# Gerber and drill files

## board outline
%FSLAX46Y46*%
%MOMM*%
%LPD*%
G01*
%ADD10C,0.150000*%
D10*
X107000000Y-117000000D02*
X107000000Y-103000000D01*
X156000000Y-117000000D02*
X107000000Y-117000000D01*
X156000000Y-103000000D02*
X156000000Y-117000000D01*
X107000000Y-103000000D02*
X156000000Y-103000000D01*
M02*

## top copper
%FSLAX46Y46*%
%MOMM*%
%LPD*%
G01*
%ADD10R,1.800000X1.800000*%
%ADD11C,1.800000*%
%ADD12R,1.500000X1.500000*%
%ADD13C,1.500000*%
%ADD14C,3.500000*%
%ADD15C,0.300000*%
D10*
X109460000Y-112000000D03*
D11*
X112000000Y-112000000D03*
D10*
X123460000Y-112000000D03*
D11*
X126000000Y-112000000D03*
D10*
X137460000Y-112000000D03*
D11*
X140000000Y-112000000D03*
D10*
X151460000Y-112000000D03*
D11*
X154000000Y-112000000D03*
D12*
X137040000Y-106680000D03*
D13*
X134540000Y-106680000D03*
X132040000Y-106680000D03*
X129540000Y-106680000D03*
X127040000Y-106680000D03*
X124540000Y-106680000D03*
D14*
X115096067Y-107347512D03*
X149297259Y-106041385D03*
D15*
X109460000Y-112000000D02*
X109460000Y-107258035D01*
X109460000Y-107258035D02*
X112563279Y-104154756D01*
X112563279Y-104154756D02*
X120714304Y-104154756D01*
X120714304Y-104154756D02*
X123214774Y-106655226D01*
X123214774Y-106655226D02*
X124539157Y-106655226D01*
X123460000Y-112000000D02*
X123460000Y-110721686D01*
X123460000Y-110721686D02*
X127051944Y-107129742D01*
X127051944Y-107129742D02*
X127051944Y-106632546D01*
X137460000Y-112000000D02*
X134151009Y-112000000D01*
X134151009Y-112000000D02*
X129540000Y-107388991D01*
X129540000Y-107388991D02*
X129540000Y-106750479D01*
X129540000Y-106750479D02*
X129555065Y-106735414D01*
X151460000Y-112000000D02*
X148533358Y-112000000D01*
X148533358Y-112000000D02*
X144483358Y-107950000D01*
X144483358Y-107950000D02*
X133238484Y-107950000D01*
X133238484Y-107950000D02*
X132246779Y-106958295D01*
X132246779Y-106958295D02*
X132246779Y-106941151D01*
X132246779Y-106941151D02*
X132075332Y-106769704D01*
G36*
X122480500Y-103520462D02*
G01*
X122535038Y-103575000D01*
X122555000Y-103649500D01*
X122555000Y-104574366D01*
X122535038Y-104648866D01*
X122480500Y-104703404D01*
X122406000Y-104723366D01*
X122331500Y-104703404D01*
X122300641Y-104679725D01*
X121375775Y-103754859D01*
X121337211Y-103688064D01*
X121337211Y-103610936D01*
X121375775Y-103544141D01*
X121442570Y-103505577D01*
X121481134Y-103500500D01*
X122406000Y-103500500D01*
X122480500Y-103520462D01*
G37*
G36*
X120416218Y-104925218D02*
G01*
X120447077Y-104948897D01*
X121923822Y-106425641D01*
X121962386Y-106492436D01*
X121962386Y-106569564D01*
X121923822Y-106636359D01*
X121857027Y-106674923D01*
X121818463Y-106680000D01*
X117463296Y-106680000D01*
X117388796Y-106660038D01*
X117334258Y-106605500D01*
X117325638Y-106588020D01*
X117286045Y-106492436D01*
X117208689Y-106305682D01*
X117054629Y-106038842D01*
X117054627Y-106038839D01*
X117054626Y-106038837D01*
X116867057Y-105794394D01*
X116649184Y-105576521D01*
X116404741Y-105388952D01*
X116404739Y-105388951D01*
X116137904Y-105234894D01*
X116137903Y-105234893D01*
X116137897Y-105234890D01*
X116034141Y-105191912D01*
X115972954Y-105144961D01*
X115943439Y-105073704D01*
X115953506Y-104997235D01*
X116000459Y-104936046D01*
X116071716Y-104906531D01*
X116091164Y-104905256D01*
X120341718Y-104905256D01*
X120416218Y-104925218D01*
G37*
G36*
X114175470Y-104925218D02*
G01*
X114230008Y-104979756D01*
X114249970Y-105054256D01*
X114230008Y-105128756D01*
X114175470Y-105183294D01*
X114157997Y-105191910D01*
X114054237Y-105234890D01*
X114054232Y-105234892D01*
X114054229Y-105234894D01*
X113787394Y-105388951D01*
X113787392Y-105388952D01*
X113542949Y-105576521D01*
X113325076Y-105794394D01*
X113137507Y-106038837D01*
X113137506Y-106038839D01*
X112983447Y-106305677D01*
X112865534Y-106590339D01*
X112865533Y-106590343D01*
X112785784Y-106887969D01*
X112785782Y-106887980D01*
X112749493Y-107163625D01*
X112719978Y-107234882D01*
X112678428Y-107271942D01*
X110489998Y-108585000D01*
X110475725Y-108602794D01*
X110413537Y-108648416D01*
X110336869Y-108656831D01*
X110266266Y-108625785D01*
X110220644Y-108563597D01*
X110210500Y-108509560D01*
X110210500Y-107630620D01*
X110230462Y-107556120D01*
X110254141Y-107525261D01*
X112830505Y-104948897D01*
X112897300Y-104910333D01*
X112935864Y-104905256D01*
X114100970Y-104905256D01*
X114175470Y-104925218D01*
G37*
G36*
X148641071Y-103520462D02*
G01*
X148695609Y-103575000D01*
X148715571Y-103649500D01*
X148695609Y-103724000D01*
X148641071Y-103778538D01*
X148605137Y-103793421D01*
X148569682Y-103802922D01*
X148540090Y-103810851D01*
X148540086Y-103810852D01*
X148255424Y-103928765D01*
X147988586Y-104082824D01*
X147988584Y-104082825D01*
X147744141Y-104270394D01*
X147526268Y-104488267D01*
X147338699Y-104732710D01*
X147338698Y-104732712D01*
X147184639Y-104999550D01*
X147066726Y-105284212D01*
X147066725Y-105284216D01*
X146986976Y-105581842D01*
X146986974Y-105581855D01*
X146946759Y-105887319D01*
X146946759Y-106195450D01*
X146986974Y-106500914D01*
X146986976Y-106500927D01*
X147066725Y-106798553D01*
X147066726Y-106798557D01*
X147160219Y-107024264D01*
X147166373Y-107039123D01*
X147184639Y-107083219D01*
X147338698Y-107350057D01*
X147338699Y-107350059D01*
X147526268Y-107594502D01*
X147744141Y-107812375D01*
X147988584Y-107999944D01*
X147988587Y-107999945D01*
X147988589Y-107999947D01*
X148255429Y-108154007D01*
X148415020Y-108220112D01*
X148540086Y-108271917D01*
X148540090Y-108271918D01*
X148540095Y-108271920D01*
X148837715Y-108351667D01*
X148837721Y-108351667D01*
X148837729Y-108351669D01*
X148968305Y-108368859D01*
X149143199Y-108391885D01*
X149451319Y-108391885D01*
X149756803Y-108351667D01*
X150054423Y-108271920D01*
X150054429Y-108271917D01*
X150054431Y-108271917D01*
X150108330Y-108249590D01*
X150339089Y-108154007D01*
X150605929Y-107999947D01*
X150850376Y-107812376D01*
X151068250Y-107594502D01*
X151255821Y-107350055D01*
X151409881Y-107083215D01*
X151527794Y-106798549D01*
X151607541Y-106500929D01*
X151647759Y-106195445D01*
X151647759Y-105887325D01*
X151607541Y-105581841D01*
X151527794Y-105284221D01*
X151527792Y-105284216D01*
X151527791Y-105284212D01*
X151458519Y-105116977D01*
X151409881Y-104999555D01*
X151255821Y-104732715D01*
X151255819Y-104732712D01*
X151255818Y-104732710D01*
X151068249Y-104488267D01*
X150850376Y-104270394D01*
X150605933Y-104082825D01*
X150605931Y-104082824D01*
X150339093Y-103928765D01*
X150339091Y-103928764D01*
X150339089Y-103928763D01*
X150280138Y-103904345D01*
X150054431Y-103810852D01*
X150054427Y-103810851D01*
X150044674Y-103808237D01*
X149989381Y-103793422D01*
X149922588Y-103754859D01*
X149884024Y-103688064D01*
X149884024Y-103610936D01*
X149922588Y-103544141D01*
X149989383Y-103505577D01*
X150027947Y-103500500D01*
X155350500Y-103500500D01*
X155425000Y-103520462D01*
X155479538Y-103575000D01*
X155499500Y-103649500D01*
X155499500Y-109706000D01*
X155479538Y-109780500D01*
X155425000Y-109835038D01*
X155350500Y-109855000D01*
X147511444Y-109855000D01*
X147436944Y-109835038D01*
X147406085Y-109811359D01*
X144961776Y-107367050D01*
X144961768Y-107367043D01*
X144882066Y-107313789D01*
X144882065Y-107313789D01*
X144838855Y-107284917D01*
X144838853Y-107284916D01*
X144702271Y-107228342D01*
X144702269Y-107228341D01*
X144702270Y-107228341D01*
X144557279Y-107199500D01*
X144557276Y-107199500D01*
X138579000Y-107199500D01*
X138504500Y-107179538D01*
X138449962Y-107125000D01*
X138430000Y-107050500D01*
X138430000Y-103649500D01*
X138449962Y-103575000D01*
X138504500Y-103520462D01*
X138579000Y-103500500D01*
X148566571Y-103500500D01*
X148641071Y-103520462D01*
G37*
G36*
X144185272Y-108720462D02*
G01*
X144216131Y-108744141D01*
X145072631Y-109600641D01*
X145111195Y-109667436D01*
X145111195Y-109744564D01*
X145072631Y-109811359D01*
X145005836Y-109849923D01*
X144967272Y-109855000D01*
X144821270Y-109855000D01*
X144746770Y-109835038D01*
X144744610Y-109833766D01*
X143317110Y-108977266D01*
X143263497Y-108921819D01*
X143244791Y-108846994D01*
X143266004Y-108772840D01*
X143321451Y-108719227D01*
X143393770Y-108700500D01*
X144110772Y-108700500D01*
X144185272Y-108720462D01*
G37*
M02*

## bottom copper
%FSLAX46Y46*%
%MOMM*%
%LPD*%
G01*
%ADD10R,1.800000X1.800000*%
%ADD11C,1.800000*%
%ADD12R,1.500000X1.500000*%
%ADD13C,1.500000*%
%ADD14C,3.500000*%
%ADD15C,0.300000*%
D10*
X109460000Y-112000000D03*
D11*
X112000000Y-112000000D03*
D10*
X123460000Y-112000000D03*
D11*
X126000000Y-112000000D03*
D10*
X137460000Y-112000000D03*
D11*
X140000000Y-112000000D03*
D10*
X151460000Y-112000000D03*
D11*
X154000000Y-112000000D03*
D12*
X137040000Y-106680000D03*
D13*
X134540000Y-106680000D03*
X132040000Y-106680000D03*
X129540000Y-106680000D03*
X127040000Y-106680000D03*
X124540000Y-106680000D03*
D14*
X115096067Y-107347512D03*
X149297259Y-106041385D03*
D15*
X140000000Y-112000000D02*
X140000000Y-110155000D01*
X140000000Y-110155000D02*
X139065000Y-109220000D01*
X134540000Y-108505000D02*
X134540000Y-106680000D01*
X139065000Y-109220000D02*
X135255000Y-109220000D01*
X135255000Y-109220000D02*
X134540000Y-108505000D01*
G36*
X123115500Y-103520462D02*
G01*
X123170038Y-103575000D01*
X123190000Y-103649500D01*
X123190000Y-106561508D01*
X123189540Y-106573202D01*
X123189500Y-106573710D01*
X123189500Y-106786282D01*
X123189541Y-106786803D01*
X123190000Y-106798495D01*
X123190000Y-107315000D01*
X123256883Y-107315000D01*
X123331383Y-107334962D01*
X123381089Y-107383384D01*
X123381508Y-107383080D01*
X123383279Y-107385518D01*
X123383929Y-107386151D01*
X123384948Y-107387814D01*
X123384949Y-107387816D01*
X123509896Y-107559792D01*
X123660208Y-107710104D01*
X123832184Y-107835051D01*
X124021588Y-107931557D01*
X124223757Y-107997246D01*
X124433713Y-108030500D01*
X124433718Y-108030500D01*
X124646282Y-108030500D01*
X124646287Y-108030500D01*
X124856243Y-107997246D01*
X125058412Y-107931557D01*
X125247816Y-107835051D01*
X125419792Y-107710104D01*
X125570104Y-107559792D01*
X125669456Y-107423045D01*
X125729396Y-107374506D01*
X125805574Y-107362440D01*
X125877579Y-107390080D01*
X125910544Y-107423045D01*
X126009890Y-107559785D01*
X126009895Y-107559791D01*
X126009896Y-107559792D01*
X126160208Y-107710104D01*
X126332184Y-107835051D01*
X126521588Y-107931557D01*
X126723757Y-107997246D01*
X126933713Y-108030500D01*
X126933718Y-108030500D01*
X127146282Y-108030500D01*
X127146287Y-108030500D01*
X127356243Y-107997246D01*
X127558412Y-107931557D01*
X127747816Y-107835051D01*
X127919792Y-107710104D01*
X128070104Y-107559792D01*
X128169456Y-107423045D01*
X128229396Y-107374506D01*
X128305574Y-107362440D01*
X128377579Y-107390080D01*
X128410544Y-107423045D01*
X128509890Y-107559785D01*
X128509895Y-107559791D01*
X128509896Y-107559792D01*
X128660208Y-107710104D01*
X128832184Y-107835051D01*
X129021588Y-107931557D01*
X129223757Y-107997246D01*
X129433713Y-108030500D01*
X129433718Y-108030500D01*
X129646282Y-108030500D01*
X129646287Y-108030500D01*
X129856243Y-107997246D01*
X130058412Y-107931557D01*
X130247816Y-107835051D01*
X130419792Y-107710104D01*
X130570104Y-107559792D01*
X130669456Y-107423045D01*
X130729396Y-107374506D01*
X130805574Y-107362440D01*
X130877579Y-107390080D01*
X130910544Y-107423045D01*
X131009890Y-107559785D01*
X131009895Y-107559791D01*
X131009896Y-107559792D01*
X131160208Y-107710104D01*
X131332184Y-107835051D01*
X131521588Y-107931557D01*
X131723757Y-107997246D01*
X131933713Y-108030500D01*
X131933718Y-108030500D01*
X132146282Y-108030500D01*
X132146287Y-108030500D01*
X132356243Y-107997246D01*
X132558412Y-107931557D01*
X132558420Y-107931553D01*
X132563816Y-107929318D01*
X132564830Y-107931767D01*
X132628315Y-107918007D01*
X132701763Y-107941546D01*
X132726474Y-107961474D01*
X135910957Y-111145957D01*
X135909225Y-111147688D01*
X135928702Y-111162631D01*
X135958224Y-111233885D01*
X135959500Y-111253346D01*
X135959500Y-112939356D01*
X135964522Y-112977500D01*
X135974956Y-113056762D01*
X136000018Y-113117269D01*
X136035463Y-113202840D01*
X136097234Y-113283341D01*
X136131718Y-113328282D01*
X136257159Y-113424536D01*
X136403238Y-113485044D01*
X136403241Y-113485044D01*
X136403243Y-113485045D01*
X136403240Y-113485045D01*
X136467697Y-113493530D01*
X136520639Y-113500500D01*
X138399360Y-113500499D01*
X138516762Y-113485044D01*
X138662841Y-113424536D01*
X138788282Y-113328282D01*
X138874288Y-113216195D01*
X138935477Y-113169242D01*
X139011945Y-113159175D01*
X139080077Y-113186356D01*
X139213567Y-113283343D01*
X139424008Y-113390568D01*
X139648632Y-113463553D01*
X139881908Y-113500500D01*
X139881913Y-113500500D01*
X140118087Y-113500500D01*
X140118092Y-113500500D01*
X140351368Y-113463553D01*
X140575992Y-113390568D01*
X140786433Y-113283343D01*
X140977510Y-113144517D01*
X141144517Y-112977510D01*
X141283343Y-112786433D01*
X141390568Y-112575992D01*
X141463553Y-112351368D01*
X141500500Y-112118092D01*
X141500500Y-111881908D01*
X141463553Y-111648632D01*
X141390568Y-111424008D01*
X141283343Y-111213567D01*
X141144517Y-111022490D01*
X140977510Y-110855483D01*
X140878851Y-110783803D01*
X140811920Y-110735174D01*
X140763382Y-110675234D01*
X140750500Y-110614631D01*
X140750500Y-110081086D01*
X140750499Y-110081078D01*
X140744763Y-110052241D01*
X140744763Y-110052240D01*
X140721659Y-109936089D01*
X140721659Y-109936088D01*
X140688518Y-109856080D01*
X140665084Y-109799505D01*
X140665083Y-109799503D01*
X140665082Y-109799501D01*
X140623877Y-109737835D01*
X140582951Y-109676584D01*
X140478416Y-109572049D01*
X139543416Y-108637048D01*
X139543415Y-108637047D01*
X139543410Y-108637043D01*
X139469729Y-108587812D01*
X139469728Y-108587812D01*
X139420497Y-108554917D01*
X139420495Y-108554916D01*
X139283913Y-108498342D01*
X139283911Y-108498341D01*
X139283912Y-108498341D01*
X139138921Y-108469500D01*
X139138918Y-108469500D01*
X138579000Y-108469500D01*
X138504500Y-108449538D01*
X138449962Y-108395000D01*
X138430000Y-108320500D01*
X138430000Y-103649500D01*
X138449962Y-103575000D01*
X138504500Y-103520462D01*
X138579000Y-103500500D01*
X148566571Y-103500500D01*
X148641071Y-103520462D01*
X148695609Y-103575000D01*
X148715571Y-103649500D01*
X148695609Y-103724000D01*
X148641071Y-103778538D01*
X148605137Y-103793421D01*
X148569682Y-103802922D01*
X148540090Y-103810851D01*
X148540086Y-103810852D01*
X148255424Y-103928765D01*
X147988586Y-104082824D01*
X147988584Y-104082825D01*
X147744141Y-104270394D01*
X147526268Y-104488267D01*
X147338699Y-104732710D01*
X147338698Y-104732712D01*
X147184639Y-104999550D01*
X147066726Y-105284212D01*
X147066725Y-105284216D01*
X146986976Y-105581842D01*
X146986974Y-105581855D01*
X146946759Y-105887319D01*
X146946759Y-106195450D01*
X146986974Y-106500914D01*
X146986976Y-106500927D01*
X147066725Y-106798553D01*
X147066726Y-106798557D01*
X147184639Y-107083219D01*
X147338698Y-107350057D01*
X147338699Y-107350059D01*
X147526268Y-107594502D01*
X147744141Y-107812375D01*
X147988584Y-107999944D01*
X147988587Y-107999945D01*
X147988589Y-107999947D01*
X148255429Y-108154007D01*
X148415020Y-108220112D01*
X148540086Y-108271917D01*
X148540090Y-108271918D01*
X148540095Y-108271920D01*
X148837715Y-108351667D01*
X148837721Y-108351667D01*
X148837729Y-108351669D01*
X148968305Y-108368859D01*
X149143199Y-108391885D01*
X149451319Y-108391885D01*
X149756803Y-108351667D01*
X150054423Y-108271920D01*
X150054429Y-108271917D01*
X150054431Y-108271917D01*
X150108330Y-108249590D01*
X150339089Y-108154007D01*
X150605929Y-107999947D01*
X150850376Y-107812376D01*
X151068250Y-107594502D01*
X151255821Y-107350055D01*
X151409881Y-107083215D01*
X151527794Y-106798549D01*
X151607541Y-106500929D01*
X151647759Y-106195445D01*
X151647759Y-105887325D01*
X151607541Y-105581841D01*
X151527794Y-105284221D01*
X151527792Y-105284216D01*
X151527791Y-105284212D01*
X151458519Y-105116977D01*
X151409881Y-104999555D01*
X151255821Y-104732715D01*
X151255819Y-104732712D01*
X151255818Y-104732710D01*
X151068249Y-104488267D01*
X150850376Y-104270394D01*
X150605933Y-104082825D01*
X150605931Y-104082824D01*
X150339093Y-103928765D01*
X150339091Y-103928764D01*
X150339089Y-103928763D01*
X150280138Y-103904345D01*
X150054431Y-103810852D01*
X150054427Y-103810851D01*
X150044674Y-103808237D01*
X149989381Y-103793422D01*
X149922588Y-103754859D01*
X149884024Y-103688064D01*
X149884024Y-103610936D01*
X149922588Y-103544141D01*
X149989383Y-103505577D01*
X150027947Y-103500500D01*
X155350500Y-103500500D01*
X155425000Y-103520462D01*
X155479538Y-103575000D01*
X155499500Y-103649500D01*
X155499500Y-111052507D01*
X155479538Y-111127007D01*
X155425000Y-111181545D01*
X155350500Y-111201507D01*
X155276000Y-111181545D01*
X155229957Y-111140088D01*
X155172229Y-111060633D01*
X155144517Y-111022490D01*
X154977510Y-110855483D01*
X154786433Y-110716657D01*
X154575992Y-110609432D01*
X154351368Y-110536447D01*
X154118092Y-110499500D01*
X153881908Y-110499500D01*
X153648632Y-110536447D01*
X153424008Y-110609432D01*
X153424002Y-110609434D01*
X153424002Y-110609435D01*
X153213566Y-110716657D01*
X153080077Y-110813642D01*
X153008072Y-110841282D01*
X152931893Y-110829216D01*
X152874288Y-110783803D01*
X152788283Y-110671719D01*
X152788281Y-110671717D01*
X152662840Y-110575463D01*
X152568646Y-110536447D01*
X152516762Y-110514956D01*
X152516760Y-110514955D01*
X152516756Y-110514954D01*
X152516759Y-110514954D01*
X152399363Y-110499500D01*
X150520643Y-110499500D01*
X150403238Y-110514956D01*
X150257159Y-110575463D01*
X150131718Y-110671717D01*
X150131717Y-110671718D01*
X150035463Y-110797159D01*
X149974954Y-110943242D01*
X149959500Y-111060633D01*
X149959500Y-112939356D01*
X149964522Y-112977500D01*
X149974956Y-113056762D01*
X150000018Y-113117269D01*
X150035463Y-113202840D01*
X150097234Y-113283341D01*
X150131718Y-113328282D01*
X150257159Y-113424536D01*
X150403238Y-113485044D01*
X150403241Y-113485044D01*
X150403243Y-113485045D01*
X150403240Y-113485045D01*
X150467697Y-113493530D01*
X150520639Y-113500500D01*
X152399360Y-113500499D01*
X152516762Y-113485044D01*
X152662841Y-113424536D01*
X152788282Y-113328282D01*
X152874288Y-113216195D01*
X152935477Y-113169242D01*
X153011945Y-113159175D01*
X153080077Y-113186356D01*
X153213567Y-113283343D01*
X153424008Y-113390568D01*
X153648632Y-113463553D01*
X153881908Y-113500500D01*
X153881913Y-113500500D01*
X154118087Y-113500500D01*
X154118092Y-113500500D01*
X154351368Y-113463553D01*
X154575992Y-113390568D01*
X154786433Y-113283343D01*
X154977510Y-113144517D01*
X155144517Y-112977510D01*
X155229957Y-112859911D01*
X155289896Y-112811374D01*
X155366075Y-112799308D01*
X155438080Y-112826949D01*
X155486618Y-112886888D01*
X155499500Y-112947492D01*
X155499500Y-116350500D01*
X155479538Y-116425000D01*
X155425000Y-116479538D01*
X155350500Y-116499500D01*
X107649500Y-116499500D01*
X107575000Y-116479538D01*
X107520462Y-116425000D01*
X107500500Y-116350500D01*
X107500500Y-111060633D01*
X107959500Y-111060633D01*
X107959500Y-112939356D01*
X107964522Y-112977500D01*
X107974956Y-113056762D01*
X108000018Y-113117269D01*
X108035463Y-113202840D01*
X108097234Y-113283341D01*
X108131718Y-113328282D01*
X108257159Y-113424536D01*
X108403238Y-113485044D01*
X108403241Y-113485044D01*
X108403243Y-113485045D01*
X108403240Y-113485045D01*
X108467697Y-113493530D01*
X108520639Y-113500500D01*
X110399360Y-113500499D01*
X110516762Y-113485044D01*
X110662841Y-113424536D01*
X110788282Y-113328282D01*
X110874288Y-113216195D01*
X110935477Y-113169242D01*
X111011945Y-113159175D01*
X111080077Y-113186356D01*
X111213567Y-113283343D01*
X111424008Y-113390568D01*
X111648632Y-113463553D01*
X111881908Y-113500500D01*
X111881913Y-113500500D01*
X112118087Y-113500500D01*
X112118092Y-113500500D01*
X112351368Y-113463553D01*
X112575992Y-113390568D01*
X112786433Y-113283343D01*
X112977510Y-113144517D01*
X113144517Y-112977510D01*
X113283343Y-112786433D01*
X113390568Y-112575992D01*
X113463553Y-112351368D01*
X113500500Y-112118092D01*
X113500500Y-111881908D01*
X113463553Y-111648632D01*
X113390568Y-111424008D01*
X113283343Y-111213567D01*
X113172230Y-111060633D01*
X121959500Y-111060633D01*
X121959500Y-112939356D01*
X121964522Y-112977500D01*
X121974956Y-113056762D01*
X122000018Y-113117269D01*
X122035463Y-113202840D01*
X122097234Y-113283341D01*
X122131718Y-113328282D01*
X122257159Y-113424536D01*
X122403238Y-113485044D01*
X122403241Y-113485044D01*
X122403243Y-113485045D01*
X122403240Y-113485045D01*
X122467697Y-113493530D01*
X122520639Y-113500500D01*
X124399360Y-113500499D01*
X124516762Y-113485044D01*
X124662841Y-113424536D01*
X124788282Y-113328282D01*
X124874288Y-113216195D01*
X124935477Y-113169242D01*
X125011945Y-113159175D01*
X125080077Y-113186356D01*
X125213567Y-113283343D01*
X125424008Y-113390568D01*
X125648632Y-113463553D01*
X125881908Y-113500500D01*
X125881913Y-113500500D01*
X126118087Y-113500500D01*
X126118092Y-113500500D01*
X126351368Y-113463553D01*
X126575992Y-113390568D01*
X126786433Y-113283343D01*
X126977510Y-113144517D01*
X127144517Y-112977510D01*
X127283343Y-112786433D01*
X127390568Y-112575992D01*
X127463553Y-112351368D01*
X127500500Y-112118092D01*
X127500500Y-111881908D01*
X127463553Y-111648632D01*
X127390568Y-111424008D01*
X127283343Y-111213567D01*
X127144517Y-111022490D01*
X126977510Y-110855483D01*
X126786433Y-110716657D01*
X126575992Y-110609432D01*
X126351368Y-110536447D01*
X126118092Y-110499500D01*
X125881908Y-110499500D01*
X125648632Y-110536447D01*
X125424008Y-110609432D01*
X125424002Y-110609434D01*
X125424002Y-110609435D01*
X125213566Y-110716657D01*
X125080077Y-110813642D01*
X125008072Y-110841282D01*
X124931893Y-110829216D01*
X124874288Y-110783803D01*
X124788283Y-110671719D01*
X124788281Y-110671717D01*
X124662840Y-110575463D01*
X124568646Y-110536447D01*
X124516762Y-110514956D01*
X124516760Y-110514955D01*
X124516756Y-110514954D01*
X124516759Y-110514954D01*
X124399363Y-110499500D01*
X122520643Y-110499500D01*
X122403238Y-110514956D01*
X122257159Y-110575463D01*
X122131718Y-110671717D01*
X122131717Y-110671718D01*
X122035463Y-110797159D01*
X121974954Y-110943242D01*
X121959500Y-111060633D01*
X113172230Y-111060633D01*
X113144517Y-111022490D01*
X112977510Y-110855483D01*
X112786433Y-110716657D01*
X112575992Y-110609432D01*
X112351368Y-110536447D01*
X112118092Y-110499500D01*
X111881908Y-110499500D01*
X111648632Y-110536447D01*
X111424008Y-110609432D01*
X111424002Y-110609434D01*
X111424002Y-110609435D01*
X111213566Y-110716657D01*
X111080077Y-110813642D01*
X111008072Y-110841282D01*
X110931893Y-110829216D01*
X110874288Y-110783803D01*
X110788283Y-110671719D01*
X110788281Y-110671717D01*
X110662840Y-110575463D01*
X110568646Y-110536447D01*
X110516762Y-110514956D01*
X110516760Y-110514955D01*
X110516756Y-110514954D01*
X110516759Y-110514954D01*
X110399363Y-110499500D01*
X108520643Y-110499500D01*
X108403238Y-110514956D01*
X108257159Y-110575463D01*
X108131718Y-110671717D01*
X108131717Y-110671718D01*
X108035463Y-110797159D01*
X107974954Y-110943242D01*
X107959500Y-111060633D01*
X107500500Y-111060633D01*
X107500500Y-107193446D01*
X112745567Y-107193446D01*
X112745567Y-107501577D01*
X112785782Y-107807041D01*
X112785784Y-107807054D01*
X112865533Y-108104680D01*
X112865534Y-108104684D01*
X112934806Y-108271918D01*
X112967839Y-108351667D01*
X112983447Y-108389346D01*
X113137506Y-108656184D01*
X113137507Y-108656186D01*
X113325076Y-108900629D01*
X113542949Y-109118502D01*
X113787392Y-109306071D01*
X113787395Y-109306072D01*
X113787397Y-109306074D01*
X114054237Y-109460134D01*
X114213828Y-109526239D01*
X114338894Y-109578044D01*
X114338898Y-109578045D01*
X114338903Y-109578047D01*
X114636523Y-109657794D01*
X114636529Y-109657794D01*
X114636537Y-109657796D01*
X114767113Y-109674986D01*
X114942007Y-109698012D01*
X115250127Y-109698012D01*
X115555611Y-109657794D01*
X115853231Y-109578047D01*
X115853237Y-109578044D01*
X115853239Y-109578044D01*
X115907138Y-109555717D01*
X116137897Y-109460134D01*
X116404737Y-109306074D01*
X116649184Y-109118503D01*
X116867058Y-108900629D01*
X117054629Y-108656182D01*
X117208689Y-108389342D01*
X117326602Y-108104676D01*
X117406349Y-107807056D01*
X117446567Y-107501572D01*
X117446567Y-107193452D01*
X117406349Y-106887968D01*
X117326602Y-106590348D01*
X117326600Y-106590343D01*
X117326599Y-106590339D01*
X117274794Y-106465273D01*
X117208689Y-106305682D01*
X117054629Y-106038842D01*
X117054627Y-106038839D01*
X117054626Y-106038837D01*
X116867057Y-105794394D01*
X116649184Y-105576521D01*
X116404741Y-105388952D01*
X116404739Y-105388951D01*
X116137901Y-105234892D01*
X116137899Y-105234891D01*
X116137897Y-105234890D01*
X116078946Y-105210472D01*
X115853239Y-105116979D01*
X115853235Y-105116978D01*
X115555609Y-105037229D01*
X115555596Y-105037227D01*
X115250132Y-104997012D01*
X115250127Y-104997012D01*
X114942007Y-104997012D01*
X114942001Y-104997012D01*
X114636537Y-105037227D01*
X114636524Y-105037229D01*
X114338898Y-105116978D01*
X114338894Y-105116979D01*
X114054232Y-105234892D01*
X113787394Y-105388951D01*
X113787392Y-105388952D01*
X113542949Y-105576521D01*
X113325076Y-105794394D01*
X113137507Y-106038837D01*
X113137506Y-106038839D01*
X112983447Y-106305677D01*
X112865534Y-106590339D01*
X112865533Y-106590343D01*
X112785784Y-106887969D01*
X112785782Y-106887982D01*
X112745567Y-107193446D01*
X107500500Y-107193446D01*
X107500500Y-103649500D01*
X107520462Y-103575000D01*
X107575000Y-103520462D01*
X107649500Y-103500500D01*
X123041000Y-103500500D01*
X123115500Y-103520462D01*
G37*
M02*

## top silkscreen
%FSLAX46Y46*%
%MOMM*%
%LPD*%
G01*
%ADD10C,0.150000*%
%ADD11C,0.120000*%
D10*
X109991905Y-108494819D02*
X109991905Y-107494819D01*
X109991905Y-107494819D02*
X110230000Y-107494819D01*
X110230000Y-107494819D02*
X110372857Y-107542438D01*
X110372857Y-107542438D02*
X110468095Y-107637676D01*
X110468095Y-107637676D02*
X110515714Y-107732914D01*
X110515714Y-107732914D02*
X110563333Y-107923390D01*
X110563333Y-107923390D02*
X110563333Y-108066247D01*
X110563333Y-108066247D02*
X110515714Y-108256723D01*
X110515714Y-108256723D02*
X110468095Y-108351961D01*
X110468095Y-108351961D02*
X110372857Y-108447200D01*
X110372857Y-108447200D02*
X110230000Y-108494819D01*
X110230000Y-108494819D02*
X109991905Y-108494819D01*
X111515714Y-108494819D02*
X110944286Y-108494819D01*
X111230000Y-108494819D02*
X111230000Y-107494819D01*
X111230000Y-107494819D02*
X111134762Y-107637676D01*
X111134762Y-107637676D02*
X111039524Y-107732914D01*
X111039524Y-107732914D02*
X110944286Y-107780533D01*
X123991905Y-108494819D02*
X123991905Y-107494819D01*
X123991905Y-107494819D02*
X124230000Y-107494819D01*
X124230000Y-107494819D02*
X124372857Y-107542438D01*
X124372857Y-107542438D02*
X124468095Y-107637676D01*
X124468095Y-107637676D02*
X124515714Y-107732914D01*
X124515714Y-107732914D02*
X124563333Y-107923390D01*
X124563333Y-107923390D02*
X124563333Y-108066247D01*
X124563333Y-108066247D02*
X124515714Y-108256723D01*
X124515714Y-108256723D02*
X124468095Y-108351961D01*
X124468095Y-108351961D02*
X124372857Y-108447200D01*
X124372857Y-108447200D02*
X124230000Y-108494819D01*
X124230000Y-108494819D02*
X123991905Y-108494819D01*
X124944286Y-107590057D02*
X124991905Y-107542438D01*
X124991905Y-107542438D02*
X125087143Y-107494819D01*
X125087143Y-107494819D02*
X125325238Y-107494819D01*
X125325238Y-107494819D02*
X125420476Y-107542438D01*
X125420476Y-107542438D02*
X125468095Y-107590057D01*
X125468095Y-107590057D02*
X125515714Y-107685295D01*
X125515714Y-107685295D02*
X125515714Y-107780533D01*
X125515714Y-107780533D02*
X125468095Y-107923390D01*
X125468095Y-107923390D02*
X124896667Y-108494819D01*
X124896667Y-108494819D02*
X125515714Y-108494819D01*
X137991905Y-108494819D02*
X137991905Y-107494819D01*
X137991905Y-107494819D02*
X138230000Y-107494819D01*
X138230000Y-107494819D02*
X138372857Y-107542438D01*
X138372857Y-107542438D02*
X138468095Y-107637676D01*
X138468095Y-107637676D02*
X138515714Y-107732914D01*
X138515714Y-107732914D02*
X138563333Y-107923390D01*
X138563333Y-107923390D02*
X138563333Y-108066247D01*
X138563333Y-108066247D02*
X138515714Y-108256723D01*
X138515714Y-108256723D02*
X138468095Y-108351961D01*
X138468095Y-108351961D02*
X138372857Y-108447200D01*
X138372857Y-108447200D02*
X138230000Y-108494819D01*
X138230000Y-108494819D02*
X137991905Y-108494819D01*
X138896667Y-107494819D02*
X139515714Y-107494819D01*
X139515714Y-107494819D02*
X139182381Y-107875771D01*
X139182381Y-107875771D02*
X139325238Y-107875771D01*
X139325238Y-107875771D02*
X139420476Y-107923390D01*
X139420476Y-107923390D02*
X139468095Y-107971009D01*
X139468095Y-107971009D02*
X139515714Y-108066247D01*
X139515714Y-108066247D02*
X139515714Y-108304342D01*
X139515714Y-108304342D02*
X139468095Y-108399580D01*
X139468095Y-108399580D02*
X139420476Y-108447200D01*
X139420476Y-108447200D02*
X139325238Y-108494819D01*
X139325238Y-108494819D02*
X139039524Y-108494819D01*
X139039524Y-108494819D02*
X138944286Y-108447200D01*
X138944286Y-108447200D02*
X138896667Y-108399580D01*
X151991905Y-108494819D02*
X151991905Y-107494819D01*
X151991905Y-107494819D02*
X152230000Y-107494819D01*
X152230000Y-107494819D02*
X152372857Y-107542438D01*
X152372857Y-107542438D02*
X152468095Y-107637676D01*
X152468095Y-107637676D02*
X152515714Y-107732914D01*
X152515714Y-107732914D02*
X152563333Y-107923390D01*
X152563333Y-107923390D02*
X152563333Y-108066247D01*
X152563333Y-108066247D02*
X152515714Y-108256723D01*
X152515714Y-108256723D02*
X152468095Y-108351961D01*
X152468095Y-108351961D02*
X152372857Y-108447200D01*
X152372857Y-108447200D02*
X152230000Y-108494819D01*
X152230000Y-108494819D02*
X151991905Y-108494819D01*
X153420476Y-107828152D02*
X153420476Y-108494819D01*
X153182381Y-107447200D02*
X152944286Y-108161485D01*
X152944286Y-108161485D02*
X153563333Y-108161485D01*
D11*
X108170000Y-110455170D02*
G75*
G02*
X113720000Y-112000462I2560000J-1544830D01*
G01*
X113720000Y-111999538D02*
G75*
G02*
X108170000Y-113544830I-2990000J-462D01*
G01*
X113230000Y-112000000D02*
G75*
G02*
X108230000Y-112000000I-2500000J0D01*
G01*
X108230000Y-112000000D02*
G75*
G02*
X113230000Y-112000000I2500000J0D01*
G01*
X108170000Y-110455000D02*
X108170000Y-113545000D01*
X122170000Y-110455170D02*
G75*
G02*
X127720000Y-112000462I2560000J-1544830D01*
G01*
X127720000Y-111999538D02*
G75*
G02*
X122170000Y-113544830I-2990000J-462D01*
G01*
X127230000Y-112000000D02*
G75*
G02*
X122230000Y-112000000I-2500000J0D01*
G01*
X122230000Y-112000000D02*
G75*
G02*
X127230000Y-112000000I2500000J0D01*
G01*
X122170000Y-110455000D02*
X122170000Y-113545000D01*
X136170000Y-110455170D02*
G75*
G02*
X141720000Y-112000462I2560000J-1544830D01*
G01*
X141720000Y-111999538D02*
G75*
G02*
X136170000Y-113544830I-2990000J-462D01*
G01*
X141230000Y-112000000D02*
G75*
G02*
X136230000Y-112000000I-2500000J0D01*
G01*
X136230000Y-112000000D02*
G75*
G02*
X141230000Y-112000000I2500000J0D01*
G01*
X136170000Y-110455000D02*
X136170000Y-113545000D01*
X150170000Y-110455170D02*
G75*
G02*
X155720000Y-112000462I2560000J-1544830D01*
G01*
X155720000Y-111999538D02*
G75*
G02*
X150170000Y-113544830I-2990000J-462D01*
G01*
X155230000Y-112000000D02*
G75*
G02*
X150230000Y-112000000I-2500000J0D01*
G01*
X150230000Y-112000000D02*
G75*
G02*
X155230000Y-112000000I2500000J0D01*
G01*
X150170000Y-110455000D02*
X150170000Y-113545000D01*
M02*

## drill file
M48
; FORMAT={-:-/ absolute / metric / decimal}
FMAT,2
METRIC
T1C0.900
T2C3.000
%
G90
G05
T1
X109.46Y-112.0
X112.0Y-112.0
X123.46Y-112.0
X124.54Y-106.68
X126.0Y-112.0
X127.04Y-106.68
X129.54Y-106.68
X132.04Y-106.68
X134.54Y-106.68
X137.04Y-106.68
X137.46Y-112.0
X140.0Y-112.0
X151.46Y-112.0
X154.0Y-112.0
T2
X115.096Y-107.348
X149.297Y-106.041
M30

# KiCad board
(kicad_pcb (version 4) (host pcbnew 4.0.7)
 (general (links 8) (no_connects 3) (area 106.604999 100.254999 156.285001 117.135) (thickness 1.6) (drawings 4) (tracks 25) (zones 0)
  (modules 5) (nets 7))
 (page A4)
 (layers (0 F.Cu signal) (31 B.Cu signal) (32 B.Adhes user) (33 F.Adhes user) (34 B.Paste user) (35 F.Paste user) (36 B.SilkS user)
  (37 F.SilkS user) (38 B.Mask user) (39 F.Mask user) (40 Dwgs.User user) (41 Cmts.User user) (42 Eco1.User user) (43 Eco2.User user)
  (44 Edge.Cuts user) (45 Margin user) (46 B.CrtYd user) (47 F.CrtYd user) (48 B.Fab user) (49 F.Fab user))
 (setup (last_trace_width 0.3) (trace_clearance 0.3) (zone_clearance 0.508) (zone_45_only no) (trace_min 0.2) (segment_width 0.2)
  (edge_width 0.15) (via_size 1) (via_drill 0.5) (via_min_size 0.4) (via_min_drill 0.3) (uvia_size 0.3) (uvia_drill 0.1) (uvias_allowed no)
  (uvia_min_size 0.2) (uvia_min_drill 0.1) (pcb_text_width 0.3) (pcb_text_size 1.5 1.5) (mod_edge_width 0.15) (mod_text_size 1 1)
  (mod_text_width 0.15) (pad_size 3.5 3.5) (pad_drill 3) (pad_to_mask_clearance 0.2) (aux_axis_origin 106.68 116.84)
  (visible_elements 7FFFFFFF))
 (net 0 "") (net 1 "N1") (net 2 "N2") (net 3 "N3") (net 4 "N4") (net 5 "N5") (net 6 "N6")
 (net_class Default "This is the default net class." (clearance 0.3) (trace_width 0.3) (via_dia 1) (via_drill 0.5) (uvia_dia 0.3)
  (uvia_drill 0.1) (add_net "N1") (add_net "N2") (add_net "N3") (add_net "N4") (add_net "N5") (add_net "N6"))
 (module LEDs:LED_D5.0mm (layer F.Cu) (at 109.46 112)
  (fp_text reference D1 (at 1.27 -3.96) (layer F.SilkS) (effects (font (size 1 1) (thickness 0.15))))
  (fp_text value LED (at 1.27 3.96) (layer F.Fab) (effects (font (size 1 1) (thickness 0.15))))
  (fp_arc (start 1.27 0) (end -1.29 -1.54483) (angle 148.9) (layer F.SilkS) (width 0.12))
  (fp_arc (start 1.27 0) (end -1.29 1.54483) (angle -148.9) (layer F.SilkS) (width 0.12))
  (fp_circle (center 1.27 0) (end 3.77 0) (layer F.SilkS) (width 0.12))
  (fp_line (start -1.29 -1.545) (end -1.29 1.545) (layer F.SilkS) (width 0.12))
  (pad 1 thru_hole rect (at 0 0) (size 1.8 1.8) (drill 0.9) (layers *.Cu *.Mask) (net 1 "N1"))
  (pad 2 thru_hole circle (at 2.54 0) (size 1.8 1.8) (drill 0.9) (layers *.Cu *.Mask) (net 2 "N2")))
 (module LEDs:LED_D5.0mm (layer F.Cu) (at 123.46 112)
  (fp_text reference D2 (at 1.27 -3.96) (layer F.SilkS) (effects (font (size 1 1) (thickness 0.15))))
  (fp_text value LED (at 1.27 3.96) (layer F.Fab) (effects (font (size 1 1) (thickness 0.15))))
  (fp_arc (start 1.27 0) (end -1.29 -1.54483) (angle 148.9) (layer F.SilkS) (width 0.12))
  (fp_arc (start 1.27 0) (end -1.29 1.54483) (angle -148.9) (layer F.SilkS) (width 0.12))
  (fp_circle (center 1.27 0) (end 3.77 0) (layer F.SilkS) (width 0.12))
  (fp_line (start -1.29 -1.545) (end -1.29 1.545) (layer F.SilkS) (width 0.12))
  (pad 1 thru_hole rect (at 0 0) (size 1.8 1.8) (drill 0.9) (layers *.Cu *.Mask) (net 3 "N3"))
  (pad 2 thru_hole circle (at 2.54 0) (size 1.8 1.8) (drill 0.9) (layers *.Cu *.Mask) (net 2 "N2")))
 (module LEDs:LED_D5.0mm (layer F.Cu) (at 137.46 112)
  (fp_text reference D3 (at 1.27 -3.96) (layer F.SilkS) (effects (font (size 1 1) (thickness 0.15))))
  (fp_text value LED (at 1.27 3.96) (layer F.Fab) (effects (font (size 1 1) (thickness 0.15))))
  (fp_arc (start 1.27 0) (end -1.29 -1.54483) (angle 148.9) (layer F.SilkS) (width 0.12))
  (fp_arc (start 1.27 0) (end -1.29 1.54483) (angle -148.9) (layer F.SilkS) (width 0.12))
  (fp_circle (center 1.27 0) (end 3.77 0) (layer F.SilkS) (width 0.12))
  (fp_line (start -1.29 -1.545) (end -1.29 1.545) (layer F.SilkS) (width 0.12))
  (pad 1 thru_hole rect (at 0 0) (size 1.8 1.8) (drill 0.9) (layers *.Cu *.Mask) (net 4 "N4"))
  (pad 2 thru_hole circle (at 2.54 0) (size 1.8 1.8) (drill 0.9) (layers *.Cu *.Mask) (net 2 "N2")))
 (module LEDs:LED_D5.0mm (layer F.Cu) (at 151.46 112)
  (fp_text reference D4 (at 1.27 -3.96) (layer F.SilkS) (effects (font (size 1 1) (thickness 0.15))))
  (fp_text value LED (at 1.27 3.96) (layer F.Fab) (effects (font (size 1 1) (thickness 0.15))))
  (fp_arc (start 1.27 0) (end -1.29 -1.54483) (angle 148.9) (layer F.SilkS) (width 0.12))
  (fp_arc (start 1.27 0) (end -1.29 1.54483) (angle -148.9) (layer F.SilkS) (width 0.12))
  (fp_circle (center 1.27 0) (end 3.77 0) (layer F.SilkS) (width 0.12))
  (fp_line (start -1.29 -1.545) (end -1.29 1.545) (layer F.SilkS) (width 0.12))
  (pad 1 thru_hole rect (at 0 0) (size 1.8 1.8) (drill 0.9) (layers *.Cu *.Mask) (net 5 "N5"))
  (pad 2 thru_hole circle (at 2.54 0) (size 1.8 1.8) (drill 0.9) (layers *.Cu *.Mask) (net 2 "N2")))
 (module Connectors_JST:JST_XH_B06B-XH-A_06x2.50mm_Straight (layer B.Cu) (at 137.04 106.68 180)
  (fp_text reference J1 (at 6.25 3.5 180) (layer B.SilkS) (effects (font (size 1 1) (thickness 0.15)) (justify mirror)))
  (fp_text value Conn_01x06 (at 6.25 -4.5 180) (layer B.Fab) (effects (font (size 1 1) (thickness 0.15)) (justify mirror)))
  (pad 1 thru_hole rect (at 0 0 180) (size 1.5 1.5) (drill 0.9) (layers *.Cu *.Mask) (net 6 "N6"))
  (pad 2 thru_hole circle (at 2.5 0 180) (size 1.5 1.5) (drill 0.9) (layers *.Cu *.Mask) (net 2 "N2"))
  (pad 3 thru_hole circle (at 5 0 180) (size 1.5 1.5) (drill 0.9) (layers *.Cu *.Mask) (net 5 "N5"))
  (pad 4 thru_hole circle (at 7.5 0 180) (size 1.5 1.5) (drill 0.9) (layers *.Cu *.Mask) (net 4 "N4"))
  (pad 5 thru_hole circle (at 10 0 180) (size 1.5 1.5) (drill 0.9) (layers *.Cu *.Mask) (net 3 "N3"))
  (pad 6 thru_hole circle (at 12.5 0 180) (size 1.5 1.5) (drill 0.9) (layers *.Cu *.Mask) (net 1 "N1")))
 (gr_line (start 107 117) (end 107 103) (layer Edge.Cuts) (width 0.15))
 (gr_line (start 156 117) (end 107 117) (layer Edge.Cuts) (width 0.15))
 (gr_line (start 156 103) (end 156 117) (layer Edge.Cuts) (width 0.15))
 (gr_line (start 107 103) (end 156 103) (layer Edge.Cuts) (width 0.15))
 (via (at 115.096067 107.347512) (size 3.5) (drill 3) (layers F.Cu B.Cu) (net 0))
 (via (at 149.297259 106.041385) (size 3.5) (drill 3) (layers F.Cu B.Cu) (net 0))
 (segment (start 109.46 112) (end 109.46 107.258035) (width 0.3) (layer F.Cu) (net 1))
 (segment (start 109.46 107.258035) (end 112.563279 104.154756) (width 0.3) (layer F.Cu) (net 1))
 (segment (start 112.563279 104.154756) (end 120.714304 104.154756) (width 0.3) (layer F.Cu) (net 1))
 (segment (start 120.714304 104.154756) (end 123.214774 106.655226) (width 0.3) (layer F.Cu) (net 1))
 (segment (start 123.214774 106.655226) (end 124.539157 106.655226) (width 0.3) (layer F.Cu) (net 1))
 (segment (start 140 112) (end 140 110.155) (width 0.3) (layer B.Cu) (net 2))
 (segment (start 140 110.155) (end 139.065 109.22) (width 0.3) (layer B.Cu) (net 2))
 (segment (start 134.54 108.505) (end 134.54 106.68) (width 0.3) (layer B.Cu) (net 2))
 (segment (start 139.065 109.22) (end 135.255 109.22) (width 0.3) (layer B.Cu) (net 2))
 (segment (start 135.255 109.22) (end 134.54 108.505) (width 0.3) (layer B.Cu) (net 2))
 (segment (start 123.46 112) (end 123.46 110.721686) (width 0.3) (layer F.Cu) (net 3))
 (segment (start 123.46 110.721686) (end 127.051944 107.129742) (width 0.3) (layer F.Cu) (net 3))
 (segment (start 127.051944 107.129742) (end 127.051944 106.632546) (width 0.3) (layer F.Cu) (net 3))
 (segment (start 137.46 112) (end 134.151009 112) (width 0.3) (layer F.Cu) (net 4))
 (segment (start 134.151009 112) (end 129.54 107.388991) (width 0.3) (layer F.Cu) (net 4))
 (segment (start 129.54 107.388991) (end 129.54 106.750479) (width 0.3) (layer F.Cu) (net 4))
 (segment (start 129.54 106.750479) (end 129.555065 106.735414) (width 0.3) (layer F.Cu) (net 4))
 (segment (start 151.46 112) (end 148.533358 112) (width 0.3) (layer F.Cu) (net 5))
 (segment (start 148.533358 112) (end 144.483358 107.95) (width 0.3) (layer F.Cu) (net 5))
 (segment (start 144.483358 107.95) (end 133.238484 107.95) (width 0.3) (layer F.Cu) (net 5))
 (segment (start 133.238484 107.95) (end 132.246779 106.958295) (width 0.3) (layer F.Cu) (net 5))
 (segment (start 132.246779 106.958295) (end 132.246779 106.941151) (width 0.3) (layer F.Cu) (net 5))
 (segment (start 132.246779 106.941151) (end 132.075332 106.769704) (width 0.3) (layer F.Cu) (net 5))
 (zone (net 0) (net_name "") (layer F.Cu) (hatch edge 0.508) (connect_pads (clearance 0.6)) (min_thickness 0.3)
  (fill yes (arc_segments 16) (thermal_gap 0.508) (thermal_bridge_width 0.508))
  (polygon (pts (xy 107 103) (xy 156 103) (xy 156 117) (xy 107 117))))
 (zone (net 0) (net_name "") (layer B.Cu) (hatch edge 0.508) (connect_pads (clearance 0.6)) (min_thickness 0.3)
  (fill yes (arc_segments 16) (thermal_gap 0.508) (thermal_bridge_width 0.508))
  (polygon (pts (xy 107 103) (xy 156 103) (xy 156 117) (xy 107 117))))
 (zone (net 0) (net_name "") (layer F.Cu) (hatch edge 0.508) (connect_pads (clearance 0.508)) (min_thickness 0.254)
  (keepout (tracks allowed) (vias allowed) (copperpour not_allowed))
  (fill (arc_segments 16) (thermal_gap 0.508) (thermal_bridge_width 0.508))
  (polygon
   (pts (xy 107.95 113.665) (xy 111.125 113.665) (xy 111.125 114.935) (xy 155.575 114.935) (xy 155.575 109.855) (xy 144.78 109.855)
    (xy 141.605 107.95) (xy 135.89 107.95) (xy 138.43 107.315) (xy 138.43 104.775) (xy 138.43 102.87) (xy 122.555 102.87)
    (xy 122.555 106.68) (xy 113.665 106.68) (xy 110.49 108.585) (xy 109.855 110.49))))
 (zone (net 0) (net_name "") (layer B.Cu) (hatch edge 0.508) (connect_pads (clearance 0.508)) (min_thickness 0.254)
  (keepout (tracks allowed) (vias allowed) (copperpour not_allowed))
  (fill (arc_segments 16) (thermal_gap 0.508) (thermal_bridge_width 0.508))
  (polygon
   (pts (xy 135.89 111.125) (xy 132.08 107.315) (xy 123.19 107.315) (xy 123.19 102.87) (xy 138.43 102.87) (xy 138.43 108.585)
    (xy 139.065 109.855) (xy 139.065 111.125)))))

